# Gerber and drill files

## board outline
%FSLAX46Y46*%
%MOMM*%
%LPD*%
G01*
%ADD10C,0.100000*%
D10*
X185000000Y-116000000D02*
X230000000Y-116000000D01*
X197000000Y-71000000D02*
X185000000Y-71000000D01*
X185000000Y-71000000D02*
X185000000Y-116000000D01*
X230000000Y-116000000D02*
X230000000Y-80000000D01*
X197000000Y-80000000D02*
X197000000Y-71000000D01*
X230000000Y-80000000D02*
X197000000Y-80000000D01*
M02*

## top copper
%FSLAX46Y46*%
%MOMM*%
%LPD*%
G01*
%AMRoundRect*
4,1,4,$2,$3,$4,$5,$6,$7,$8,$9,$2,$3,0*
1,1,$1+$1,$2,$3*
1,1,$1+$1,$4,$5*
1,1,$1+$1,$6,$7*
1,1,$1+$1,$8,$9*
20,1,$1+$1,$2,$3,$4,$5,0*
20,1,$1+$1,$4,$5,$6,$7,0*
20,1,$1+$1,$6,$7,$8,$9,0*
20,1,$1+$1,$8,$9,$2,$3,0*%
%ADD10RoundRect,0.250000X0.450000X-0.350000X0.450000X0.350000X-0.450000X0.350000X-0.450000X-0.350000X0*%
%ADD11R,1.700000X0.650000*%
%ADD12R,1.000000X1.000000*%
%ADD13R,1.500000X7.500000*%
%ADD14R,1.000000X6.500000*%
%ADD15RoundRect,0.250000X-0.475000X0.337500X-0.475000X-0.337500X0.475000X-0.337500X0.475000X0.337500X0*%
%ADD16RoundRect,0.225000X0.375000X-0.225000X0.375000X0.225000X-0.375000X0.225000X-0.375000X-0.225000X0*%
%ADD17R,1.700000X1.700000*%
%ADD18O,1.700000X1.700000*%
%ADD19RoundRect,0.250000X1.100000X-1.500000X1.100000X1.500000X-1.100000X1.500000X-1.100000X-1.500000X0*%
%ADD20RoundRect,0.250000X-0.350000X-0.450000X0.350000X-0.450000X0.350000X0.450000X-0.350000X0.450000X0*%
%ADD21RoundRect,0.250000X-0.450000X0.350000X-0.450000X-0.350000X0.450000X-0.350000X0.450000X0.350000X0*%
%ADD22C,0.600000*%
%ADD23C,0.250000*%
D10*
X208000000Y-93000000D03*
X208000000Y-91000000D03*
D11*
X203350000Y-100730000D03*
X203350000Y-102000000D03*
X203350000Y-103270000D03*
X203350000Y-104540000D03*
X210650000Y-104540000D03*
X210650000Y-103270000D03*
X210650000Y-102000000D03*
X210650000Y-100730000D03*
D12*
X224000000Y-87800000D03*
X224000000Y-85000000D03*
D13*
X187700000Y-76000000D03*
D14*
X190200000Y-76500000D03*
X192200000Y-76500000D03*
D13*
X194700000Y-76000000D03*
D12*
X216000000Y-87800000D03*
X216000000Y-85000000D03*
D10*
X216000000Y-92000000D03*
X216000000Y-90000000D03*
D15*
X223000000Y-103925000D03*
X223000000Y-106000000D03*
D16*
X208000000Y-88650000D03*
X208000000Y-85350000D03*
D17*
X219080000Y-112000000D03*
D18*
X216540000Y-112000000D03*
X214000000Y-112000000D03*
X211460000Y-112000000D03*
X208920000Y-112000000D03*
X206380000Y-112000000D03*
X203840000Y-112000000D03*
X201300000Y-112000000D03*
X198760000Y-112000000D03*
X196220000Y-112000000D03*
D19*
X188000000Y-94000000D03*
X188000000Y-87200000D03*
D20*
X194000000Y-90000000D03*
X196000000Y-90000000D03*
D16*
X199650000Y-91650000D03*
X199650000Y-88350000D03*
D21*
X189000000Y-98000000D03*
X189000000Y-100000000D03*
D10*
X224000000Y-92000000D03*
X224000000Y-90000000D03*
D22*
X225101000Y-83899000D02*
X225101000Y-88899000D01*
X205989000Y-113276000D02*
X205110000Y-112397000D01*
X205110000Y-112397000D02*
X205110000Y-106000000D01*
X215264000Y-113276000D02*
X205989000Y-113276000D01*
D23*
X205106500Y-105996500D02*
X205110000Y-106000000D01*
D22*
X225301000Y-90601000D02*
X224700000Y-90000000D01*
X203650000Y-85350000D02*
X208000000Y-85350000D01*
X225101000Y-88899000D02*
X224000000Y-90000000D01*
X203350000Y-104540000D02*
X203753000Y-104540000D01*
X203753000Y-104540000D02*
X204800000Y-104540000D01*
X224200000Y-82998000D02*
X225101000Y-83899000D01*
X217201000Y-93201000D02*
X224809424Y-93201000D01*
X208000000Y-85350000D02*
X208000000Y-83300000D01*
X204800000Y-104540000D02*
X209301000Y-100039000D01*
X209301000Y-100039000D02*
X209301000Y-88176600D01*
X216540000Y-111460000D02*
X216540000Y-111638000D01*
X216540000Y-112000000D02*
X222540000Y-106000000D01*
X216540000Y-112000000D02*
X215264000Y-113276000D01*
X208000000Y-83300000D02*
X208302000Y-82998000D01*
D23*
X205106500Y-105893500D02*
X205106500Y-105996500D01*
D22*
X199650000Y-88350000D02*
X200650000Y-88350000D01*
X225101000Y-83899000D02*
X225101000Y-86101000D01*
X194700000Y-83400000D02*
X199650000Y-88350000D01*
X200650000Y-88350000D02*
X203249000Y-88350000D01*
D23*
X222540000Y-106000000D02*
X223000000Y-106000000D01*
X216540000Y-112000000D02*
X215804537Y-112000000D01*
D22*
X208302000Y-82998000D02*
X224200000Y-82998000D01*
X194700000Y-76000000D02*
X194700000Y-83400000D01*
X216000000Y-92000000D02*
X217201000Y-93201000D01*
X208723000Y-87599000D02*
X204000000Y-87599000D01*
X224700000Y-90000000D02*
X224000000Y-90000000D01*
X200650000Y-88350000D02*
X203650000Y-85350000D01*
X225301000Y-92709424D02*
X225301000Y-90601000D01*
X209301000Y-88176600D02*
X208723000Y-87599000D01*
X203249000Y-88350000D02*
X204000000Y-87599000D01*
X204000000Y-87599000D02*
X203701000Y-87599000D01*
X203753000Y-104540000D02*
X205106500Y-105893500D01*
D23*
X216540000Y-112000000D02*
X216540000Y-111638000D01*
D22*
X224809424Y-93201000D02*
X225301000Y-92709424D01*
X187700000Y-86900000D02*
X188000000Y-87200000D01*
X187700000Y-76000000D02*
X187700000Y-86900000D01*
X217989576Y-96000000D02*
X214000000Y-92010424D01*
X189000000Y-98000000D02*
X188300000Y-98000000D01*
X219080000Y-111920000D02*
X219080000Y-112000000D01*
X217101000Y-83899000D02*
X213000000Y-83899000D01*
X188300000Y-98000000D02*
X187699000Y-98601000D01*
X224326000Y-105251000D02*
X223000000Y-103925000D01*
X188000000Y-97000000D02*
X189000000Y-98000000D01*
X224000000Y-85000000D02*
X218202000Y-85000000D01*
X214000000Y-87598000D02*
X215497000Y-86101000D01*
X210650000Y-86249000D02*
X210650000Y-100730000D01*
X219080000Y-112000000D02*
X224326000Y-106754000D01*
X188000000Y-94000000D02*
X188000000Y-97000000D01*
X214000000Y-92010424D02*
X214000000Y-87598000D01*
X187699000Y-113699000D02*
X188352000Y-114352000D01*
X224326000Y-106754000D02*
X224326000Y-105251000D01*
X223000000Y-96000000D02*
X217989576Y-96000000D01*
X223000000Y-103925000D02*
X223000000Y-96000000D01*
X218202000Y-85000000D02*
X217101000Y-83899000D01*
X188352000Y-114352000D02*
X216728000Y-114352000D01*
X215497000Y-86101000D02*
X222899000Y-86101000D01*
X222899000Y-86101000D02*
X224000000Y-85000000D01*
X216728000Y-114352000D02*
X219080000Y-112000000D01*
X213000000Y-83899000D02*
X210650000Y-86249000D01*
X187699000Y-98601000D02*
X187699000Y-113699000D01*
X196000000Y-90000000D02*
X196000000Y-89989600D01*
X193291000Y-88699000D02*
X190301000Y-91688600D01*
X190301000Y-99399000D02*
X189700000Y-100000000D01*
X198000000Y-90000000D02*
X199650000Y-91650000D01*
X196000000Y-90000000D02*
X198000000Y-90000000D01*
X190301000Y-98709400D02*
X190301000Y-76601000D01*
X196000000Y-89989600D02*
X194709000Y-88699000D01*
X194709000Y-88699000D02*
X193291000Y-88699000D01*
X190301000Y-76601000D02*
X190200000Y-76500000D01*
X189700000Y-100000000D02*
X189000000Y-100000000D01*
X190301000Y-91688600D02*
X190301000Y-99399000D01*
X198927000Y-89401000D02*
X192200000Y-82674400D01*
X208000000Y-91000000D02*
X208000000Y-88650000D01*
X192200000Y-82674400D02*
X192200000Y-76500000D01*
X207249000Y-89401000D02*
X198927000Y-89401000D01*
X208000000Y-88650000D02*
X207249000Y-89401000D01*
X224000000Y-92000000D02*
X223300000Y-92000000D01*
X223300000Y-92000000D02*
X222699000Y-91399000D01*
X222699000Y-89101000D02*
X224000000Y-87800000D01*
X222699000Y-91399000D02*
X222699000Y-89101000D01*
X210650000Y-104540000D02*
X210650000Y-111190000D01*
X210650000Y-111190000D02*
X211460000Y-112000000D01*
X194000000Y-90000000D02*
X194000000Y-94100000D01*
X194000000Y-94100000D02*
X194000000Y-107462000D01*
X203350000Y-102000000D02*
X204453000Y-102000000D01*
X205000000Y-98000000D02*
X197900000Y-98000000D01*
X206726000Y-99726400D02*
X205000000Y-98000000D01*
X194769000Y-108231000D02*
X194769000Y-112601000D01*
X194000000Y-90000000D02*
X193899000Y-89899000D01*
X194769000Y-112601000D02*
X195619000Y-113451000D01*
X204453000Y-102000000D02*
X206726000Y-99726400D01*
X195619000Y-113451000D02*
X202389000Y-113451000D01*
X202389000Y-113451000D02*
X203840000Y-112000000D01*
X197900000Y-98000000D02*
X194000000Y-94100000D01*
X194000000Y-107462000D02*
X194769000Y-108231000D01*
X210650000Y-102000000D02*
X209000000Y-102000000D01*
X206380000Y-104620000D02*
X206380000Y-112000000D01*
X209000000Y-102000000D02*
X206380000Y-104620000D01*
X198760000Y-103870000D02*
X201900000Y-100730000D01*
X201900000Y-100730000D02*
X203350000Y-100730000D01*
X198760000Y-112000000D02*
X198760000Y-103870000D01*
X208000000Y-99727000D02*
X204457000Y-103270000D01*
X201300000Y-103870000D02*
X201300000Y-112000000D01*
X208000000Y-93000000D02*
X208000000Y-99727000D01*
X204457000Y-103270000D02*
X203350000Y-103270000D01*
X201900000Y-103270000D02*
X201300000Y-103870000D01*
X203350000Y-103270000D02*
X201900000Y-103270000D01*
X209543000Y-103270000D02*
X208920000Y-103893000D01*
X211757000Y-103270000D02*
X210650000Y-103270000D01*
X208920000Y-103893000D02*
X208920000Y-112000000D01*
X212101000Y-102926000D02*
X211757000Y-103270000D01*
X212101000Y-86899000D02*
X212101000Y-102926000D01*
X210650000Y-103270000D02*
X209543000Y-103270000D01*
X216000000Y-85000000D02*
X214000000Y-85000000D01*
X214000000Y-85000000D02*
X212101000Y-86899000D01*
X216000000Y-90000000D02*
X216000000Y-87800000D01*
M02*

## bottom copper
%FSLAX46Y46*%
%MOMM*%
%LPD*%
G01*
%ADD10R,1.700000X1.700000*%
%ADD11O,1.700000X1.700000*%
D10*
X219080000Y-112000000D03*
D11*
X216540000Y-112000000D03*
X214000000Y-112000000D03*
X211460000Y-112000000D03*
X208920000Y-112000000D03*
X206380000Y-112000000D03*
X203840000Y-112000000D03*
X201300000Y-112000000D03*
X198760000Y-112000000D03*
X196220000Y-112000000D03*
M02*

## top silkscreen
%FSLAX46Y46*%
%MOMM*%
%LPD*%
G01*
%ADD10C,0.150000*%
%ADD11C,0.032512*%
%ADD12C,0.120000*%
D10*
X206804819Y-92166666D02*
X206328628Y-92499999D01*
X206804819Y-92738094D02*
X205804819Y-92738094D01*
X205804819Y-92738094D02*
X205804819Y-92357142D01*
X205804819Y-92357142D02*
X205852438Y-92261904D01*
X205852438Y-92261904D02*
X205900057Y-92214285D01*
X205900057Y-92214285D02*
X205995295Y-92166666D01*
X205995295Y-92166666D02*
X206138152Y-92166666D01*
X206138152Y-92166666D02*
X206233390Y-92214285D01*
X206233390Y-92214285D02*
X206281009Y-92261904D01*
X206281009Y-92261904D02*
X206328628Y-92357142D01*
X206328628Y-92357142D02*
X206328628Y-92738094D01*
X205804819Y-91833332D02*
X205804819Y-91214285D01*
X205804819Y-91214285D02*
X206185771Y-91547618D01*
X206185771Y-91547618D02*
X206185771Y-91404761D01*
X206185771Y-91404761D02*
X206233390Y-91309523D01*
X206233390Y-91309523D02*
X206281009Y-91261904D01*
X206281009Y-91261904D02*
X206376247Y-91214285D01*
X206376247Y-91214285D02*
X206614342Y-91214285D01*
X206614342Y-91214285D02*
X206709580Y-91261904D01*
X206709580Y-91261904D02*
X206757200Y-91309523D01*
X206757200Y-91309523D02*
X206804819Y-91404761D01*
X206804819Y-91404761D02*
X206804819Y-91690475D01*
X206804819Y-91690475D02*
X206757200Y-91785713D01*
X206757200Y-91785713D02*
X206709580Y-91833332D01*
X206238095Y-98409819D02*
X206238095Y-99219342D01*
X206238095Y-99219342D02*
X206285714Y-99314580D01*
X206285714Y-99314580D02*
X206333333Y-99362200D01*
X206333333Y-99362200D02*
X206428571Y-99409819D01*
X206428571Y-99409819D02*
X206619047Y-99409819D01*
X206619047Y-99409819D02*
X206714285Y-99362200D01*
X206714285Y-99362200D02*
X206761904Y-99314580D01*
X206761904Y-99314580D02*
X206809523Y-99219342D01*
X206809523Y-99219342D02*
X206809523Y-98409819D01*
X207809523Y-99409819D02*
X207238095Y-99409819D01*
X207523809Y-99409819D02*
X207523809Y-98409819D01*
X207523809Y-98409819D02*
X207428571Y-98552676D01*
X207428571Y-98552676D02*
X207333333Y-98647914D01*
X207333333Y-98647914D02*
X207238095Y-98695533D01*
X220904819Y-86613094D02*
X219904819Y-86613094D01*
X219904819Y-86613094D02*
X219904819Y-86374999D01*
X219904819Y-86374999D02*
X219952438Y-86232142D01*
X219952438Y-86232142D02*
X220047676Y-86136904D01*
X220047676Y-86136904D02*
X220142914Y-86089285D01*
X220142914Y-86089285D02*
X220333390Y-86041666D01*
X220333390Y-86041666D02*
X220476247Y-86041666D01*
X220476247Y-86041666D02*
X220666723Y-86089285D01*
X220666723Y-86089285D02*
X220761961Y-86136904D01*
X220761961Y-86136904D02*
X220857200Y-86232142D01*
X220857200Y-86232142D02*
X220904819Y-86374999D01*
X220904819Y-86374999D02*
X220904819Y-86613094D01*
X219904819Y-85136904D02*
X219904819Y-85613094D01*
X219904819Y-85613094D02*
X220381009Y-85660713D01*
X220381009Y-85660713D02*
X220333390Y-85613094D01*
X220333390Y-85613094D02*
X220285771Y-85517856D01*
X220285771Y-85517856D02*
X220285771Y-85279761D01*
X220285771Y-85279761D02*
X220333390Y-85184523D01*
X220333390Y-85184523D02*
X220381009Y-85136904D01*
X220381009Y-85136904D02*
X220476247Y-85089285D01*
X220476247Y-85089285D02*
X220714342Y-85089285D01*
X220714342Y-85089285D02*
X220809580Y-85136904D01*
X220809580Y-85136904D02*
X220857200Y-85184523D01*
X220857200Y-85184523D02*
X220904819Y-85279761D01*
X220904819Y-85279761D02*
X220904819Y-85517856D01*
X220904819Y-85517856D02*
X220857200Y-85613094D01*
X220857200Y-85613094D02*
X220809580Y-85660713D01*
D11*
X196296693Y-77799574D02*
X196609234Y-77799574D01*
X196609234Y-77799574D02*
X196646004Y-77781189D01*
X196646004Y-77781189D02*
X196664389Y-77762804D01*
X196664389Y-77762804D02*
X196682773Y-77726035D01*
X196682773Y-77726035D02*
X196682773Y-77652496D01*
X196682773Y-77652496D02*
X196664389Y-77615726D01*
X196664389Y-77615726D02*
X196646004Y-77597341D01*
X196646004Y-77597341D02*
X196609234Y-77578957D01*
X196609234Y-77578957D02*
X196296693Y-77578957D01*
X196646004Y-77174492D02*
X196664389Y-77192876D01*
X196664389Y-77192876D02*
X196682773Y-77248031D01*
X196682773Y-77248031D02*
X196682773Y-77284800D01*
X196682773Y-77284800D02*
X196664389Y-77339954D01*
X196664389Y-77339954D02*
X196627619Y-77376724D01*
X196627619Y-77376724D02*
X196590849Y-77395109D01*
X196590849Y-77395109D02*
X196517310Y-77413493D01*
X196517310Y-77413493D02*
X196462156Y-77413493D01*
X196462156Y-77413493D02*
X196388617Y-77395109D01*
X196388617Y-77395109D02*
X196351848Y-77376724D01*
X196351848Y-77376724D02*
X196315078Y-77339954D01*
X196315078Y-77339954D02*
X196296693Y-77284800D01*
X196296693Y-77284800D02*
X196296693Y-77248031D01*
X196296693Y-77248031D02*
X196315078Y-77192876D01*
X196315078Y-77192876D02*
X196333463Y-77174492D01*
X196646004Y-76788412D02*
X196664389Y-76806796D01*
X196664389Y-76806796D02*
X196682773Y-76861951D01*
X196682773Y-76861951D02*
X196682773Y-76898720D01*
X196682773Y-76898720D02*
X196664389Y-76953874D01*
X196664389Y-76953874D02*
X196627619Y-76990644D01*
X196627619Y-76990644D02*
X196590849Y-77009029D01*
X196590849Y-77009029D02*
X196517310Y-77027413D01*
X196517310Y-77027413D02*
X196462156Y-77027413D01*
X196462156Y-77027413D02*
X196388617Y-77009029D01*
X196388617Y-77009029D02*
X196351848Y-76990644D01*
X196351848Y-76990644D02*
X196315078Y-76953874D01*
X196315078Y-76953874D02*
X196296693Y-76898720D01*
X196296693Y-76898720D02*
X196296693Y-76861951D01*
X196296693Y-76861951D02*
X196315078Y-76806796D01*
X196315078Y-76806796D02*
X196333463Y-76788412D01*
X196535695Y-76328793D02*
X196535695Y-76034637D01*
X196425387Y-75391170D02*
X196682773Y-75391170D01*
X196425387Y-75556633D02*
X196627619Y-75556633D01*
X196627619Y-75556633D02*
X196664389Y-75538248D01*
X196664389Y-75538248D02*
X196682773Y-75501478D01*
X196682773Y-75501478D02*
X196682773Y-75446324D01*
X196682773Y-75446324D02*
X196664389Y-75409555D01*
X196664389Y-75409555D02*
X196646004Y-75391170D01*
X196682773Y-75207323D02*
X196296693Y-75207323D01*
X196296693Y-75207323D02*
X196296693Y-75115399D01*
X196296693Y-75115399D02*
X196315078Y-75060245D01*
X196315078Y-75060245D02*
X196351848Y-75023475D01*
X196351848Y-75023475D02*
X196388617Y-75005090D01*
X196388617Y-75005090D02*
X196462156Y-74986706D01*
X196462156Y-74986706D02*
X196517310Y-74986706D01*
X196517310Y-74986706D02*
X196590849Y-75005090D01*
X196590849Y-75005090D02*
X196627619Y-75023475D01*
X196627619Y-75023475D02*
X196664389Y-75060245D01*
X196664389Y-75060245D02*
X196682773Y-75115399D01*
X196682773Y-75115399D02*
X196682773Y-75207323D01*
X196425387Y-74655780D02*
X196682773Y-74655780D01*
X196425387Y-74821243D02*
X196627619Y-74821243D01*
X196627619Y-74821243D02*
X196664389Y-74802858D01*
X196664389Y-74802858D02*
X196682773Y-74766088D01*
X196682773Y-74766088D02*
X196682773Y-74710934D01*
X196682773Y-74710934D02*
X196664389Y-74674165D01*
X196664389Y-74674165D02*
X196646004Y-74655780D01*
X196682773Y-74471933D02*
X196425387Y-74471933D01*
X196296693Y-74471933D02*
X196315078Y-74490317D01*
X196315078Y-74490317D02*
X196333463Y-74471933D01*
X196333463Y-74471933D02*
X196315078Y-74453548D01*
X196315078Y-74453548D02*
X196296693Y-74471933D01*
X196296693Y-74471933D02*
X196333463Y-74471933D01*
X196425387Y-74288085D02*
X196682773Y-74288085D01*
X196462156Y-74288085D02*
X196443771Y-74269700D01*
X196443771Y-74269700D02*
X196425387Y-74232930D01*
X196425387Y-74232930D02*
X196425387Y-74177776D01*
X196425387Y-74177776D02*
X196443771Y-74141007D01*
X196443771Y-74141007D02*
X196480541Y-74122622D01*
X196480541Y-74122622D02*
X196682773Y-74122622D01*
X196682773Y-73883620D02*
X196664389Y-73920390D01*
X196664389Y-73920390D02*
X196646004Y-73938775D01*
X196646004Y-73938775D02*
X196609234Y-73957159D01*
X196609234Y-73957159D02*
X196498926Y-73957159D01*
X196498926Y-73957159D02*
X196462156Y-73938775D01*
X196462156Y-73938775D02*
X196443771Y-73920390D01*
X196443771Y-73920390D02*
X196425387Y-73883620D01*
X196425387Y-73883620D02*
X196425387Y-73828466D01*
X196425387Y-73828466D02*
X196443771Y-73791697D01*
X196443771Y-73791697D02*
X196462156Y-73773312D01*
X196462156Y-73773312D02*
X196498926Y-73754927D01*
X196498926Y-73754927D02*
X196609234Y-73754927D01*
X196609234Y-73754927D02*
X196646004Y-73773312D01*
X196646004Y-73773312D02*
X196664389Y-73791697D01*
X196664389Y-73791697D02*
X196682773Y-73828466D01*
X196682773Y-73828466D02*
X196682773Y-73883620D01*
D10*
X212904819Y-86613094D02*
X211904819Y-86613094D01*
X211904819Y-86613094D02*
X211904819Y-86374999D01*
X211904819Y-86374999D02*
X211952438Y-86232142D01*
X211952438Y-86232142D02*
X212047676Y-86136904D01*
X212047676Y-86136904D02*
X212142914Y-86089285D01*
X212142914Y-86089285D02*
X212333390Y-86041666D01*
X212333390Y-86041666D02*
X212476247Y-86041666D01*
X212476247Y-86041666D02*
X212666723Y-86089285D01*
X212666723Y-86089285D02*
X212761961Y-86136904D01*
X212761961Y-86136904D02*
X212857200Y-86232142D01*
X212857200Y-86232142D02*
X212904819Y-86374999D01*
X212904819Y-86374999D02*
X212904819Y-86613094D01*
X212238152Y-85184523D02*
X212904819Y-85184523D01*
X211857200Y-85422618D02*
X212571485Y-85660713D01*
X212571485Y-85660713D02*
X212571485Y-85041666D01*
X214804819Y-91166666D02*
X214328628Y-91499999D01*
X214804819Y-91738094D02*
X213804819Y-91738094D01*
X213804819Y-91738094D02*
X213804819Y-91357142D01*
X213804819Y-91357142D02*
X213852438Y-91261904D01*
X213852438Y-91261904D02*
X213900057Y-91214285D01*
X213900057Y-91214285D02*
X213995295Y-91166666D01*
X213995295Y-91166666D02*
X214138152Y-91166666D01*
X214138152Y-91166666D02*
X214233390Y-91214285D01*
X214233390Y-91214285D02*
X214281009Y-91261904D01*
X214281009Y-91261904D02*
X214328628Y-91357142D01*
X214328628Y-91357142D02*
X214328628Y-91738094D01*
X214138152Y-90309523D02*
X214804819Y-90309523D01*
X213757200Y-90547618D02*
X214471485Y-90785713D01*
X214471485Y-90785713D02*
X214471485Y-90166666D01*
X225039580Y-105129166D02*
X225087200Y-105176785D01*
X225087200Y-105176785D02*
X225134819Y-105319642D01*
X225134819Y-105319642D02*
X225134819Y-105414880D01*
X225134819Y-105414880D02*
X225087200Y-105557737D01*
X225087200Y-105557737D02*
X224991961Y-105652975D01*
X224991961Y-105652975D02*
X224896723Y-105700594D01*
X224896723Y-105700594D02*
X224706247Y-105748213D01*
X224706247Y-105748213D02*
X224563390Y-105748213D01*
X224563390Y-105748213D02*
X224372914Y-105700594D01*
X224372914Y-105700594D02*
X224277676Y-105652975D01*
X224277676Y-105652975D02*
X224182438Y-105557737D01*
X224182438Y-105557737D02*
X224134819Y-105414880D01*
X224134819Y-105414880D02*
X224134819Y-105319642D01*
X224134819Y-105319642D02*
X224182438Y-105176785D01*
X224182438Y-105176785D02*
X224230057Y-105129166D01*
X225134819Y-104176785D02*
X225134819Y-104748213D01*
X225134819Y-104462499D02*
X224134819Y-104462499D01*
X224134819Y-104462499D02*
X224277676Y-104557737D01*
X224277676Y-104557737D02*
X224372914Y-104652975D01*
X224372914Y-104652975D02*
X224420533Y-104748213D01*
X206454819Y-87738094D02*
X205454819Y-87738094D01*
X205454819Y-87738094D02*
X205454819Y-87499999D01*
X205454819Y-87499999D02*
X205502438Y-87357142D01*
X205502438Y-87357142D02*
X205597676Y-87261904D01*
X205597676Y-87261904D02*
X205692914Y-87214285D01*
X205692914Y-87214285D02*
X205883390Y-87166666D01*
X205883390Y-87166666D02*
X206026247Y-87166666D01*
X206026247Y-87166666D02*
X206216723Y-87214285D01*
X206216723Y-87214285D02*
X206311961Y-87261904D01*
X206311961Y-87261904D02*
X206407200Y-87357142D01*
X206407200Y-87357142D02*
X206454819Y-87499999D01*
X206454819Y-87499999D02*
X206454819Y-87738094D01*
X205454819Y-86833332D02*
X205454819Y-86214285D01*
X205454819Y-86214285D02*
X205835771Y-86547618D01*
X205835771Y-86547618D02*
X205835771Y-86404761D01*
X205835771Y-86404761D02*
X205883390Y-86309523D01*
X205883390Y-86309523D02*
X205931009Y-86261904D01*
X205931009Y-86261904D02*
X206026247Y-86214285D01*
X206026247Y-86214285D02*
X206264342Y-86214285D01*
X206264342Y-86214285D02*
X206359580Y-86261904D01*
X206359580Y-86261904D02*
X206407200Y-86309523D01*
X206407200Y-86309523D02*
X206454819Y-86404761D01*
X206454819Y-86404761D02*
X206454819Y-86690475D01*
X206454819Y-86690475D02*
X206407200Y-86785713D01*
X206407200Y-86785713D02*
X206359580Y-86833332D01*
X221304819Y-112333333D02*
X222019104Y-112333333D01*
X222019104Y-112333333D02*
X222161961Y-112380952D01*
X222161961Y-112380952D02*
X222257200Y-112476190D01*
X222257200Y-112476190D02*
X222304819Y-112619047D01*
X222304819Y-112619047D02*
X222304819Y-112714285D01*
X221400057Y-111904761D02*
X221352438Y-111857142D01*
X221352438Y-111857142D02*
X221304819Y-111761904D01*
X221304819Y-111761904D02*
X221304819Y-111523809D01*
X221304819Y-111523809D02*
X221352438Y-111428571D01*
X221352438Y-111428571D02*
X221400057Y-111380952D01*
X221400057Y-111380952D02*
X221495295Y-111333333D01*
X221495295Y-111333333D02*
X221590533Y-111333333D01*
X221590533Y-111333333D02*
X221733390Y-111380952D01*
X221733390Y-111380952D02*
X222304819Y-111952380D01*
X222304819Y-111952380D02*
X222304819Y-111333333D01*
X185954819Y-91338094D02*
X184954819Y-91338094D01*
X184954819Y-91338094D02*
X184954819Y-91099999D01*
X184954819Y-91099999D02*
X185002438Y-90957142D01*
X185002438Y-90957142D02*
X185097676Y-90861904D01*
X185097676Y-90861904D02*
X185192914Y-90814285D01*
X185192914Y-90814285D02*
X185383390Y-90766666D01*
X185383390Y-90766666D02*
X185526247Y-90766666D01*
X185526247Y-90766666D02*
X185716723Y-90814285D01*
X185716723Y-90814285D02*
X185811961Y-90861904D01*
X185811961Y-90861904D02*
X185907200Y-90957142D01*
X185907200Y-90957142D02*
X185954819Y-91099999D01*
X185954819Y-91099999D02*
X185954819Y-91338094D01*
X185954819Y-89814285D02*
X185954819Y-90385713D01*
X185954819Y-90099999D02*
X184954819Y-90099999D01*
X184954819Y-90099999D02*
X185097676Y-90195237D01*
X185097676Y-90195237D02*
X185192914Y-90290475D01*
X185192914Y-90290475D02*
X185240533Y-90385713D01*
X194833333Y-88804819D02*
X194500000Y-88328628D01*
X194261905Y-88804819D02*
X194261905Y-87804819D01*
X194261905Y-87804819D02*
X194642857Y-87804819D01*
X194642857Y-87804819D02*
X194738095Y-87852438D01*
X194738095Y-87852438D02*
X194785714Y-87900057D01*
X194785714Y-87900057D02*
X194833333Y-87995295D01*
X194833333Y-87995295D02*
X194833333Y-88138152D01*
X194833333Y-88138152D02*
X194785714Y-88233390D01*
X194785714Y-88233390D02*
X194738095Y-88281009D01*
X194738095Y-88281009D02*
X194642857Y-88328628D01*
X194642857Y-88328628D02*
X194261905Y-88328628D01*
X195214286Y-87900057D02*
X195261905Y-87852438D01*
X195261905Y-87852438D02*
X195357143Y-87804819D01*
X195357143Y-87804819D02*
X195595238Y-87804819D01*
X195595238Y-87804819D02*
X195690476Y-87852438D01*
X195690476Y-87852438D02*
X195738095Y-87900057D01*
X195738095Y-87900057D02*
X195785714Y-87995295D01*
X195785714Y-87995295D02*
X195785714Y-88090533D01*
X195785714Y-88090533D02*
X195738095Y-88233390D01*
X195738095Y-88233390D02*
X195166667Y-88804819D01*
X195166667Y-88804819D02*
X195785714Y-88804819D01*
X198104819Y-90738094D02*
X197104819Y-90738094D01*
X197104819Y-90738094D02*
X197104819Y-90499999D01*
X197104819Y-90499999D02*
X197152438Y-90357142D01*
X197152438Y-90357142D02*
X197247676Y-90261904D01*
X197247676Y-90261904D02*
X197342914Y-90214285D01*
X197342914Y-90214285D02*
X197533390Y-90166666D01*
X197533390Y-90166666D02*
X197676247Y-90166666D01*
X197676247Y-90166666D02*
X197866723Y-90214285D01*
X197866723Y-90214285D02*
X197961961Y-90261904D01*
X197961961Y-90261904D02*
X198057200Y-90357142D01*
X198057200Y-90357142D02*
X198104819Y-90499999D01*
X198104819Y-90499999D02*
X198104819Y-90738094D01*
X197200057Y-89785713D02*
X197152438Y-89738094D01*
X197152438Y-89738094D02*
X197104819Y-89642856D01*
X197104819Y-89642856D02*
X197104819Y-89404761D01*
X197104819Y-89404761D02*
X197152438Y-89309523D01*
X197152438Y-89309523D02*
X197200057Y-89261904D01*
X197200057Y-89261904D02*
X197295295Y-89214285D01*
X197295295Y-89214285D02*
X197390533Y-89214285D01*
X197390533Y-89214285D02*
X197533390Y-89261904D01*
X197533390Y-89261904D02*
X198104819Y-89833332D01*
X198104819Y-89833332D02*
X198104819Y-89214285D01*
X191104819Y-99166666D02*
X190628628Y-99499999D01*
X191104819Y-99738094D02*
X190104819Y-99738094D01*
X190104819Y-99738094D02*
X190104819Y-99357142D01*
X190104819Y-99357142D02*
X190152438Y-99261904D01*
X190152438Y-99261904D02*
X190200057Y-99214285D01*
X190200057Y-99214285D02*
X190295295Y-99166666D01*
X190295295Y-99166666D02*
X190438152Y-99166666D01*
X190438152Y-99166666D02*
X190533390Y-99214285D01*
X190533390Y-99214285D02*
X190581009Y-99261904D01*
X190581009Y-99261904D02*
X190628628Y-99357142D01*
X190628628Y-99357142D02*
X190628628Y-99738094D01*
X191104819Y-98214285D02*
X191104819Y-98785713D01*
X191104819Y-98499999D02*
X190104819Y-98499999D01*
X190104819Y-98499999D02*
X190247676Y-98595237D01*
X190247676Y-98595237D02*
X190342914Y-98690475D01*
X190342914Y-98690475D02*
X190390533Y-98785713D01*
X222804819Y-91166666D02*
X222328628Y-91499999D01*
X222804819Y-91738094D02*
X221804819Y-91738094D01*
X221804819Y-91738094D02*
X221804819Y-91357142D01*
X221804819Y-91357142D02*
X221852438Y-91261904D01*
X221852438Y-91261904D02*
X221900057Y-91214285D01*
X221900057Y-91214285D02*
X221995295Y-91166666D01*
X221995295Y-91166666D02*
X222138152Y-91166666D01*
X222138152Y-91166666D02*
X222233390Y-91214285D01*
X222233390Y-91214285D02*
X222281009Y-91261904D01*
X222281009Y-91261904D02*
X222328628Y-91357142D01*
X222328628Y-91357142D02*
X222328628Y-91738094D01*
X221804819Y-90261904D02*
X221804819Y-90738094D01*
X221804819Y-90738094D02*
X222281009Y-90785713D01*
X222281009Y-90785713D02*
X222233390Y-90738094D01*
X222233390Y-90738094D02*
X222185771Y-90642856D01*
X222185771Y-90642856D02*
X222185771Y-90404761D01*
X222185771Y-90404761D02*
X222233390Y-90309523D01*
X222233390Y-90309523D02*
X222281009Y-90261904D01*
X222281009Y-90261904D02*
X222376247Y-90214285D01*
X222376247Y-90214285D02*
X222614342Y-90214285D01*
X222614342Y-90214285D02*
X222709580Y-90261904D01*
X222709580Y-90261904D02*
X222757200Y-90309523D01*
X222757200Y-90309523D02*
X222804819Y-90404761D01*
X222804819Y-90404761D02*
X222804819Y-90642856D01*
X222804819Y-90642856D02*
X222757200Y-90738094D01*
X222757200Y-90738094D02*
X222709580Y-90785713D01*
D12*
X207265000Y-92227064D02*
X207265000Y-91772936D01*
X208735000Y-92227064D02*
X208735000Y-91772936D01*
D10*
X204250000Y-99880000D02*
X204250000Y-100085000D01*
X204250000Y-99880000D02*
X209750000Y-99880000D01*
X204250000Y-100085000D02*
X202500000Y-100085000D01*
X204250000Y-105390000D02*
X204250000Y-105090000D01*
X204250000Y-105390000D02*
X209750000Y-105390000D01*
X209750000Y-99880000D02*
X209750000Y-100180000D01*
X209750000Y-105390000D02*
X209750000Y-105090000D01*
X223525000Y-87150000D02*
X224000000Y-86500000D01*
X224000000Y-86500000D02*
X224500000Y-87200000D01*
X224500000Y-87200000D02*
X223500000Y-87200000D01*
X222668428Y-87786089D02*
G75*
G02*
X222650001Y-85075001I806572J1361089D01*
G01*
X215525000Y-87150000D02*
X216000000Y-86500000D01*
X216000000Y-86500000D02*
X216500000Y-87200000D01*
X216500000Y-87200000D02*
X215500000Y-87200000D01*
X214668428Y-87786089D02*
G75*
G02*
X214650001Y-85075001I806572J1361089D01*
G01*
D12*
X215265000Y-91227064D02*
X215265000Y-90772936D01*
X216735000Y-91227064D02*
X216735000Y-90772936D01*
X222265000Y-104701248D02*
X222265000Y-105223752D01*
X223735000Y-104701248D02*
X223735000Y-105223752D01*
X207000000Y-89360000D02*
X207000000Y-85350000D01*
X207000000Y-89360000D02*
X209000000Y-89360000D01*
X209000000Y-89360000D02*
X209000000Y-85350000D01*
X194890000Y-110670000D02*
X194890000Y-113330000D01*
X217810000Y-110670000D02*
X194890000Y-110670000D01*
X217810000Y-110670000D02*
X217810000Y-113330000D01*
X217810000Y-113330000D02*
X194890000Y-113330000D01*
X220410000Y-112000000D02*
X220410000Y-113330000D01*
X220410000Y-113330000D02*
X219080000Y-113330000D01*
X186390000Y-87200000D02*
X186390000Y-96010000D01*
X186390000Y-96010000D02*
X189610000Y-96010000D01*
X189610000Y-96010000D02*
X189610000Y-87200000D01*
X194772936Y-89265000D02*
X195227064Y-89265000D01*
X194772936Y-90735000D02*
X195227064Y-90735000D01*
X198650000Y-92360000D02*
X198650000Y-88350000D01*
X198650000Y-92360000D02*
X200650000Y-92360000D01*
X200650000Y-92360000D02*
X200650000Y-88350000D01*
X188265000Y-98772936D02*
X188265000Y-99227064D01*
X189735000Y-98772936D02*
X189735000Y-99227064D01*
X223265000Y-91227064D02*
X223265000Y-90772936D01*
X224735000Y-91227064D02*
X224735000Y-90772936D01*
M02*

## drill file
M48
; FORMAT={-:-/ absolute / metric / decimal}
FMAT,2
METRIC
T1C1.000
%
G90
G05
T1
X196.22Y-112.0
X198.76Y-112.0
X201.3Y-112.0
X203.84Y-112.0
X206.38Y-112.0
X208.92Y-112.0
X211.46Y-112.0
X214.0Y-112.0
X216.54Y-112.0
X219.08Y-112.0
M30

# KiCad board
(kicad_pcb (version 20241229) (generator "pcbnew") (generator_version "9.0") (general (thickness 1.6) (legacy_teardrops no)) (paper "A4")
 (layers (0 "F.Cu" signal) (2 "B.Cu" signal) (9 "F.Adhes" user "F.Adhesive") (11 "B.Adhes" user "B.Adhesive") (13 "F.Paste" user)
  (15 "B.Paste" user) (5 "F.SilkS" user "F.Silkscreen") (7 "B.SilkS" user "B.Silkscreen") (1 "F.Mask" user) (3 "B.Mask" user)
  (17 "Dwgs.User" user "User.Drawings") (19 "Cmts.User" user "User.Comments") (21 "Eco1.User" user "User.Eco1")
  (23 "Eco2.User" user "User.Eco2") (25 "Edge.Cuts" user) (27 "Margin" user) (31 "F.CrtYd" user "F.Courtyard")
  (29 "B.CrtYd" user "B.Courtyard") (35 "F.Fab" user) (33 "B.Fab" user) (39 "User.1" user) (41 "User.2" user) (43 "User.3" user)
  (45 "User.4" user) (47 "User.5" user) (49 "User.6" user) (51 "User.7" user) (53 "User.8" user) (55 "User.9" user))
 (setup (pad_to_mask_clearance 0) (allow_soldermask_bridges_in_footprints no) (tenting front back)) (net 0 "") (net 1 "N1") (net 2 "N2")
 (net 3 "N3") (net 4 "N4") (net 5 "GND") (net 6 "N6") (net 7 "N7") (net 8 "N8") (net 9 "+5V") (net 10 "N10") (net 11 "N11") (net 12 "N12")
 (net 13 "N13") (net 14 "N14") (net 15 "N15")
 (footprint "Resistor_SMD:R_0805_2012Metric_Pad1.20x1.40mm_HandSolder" (layer "F.Cu") (at 208 92 90)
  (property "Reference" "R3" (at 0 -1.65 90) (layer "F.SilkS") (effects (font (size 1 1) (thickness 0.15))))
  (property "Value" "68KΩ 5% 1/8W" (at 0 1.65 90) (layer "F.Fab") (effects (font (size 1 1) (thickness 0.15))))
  (fp_line (start -0.227064 -0.735) (end 0.227064 -0.735) (stroke (width 0.12) (type solid)) (layer "F.SilkS"))
  (fp_line (start -0.227064 0.735) (end 0.227064 0.735) (stroke (width 0.12) (type solid)) (layer "F.SilkS"))
  (pad "1" smd roundrect (at -1 0 90) (size 1.2 1.4) (layers "F.Cu" "F.Mask" "F.Paste") (roundrect_rratio 0.208333) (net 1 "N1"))
  (pad "2" smd roundrect (at 1 0 90) (size 1.2 1.4) (layers "F.Cu" "F.Mask" "F.Paste") (roundrect_rratio 0.208333) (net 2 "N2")))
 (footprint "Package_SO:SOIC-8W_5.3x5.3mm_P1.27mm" (layer "F.Cu") (at 207 102.635)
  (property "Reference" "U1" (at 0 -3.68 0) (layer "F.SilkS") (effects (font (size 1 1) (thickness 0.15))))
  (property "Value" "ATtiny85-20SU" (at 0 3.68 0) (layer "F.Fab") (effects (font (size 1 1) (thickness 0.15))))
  (fp_line (start -2.75 -2.755) (end -2.75 -2.55) (stroke (width 0.15) (type solid)) (layer "F.SilkS"))
  (fp_line (start -2.75 -2.755) (end 2.75 -2.755) (stroke (width 0.15) (type solid)) (layer "F.SilkS"))
  (fp_line (start -2.75 -2.55) (end -4.5 -2.55) (stroke (width 0.15) (type solid)) (layer "F.SilkS"))
  (fp_line (start -2.75 2.755) (end -2.75 2.455) (stroke (width 0.15) (type solid)) (layer "F.SilkS"))
  (fp_line (start -2.75 2.755) (end 2.75 2.755) (stroke (width 0.15) (type solid)) (layer "F.SilkS"))
  (fp_line (start 2.75 -2.755) (end 2.75 -2.455) (stroke (width 0.15) (type solid)) (layer "F.SilkS"))
  (fp_line (start 2.75 2.755) (end 2.75 2.455) (stroke (width 0.15) (type solid)) (layer "F.SilkS"))
  (pad "1" smd rect (at -3.65 -1.905) (size 1.7 0.65) (layers "F.Cu" "F.Mask" "F.Paste") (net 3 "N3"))
  (pad "2" smd rect (at -3.65 -0.635) (size 1.7 0.65) (layers "F.Cu" "F.Mask" "F.Paste") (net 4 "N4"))
  (pad "3" smd rect (at -3.65 0.635) (size 1.7 0.65) (layers "F.Cu" "F.Mask" "F.Paste") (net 1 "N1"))
  (pad "4" smd rect (at -3.65 1.905) (size 1.7 0.65) (layers "F.Cu" "F.Mask" "F.Paste") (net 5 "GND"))
  (pad "5" smd rect (at 3.65 1.905) (size 1.7 0.65) (layers "F.Cu" "F.Mask" "F.Paste") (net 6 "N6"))
  (pad "6" smd rect (at 3.65 0.635) (size 1.7 0.65) (layers "F.Cu" "F.Mask" "F.Paste") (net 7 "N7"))
  (pad "7" smd rect (at 3.65 -0.635) (size 1.7 0.65) (layers "F.Cu" "F.Mask" "F.Paste") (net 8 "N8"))
  (pad "8" smd rect (at 3.65 -1.905) (size 1.7 0.65) (layers "F.Cu" "F.Mask" "F.Paste") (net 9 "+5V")))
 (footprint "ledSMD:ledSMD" (layer "F.Cu") (at 224 86 90)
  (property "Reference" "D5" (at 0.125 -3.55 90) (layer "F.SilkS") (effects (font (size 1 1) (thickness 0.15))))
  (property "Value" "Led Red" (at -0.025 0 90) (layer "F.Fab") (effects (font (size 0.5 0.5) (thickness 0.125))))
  (fp_line (start -1.15 -0.475) (end -0.5 0) (stroke (width 0.15) (type solid)) (layer "F.SilkS"))
  (fp_line (start -0.5 0) (end -1.2 0.5) (stroke (width 0.15) (type solid)) (layer "F.SilkS"))
  (fp_line (start -1.2 0.5) (end -1.2 -0.5) (stroke (width 0.15) (type solid)) (layer "F.SilkS"))
  (fp_arc (start -1.786089 -1.331572) (mid -0.435753 -2.107089) (end 0.924999 -1.349999) (stroke (width 0.15) (type solid))
   (layer "F.SilkS"))
  (pad "1" smd rect (at -1.8 0 90) (size 1 1) (layers "F.Cu" "F.Mask" "F.Paste") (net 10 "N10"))
  (pad "2" smd rect (at 1 0 90) (size 1 1) (layers "F.Cu" "F.Mask" "F.Paste") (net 9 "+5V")))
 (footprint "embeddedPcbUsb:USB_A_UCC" (layer "F.Cu") (at 191.2 76.2 -90)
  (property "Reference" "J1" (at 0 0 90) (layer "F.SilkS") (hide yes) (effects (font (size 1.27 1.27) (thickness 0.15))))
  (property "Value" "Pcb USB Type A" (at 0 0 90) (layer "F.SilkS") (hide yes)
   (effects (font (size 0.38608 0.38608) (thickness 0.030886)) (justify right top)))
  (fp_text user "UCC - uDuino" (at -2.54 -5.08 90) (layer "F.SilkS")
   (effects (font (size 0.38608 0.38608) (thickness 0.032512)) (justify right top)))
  (pad "1" smd rect (at -0.2 3.5 270) (size 7.5 1.5) (layers "F.Cu" "F.Mask" "F.Paste") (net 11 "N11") (solder_mask_margin 0.1016))
  (pad "2" smd rect (at 0.3 1 270) (size 6.5 1) (layers "F.Cu" "F.Mask" "F.Paste") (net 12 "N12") (solder_mask_margin 0.1016))
  (pad "3" smd rect (at 0.3 -1 270) (size 6.5 1) (layers "F.Cu" "F.Mask" "F.Paste") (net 2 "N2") (solder_mask_margin 0.1016))
  (pad "4" smd rect (at -0.2 -3.5 270) (size 7.5 1.5) (layers "F.Cu" "F.Mask" "F.Paste") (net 5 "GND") (solder_mask_margin 0.1016)))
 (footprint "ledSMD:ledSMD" (layer "F.Cu") (at 216 86 90)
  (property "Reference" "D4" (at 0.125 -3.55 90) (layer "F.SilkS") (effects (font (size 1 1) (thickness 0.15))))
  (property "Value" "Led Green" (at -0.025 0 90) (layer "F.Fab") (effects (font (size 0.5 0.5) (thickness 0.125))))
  (fp_line (start -1.15 -0.475) (end -0.5 0) (stroke (width 0.15) (type solid)) (layer "F.SilkS"))
  (fp_line (start -0.5 0) (end -1.2 0.5) (stroke (width 0.15) (type solid)) (layer "F.SilkS"))
  (fp_line (start -1.2 0.5) (end -1.2 -0.5) (stroke (width 0.15) (type solid)) (layer "F.SilkS"))
  (fp_arc (start -1.786089 -1.331572) (mid -0.435753 -2.107089) (end 0.924999 -1.349999) (stroke (width 0.15) (type solid))
   (layer "F.SilkS"))
  (pad "1" smd rect (at -1.8 0 90) (size 1 1) (layers "F.Cu" "F.Mask" "F.Paste") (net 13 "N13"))
  (pad "2" smd rect (at 1 0 90) (size 1 1) (layers "F.Cu" "F.Mask" "F.Paste") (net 7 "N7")))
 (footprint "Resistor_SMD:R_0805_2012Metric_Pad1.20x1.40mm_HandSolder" (layer "F.Cu") (at 216 91 90)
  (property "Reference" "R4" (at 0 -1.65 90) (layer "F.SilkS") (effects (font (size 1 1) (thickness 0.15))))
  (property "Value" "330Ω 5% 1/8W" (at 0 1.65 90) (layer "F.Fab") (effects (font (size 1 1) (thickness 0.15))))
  (fp_line (start -0.227064 -0.735) (end 0.227064 -0.735) (stroke (width 0.12) (type solid)) (layer "F.SilkS"))
  (fp_line (start -0.227064 0.735) (end 0.227064 0.735) (stroke (width 0.12) (type solid)) (layer "F.SilkS"))
  (pad "1" smd roundrect (at -1 0 90) (size 1.2 1.4) (layers "F.Cu" "F.Mask" "F.Paste") (roundrect_rratio 0.208333) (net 5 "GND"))
  (pad "2" smd roundrect (at 1 0 90) (size 1.2 1.4) (layers "F.Cu" "F.Mask" "F.Paste") (roundrect_rratio 0.208333) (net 13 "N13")))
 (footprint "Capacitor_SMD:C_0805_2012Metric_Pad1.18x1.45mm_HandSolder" (layer "F.Cu") (at 223 104.9625 -90)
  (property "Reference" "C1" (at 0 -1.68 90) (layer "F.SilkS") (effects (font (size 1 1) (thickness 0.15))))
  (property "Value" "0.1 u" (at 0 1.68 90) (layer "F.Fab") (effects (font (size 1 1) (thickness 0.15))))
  (fp_line (start -0.261252 0.735) (end 0.261252 0.735) (stroke (width 0.12) (type solid)) (layer "F.SilkS"))
  (fp_line (start -0.261252 -0.735) (end 0.261252 -0.735) (stroke (width 0.12) (type solid)) (layer "F.SilkS"))
  (pad "1" smd roundrect (at -1.0375 0 270) (size 1.175 1.45) (layers "F.Cu" "F.Mask" "F.Paste") (roundrect_rratio 0.212766) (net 9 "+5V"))
  (pad "2" smd roundrect (at 1.0375 0 270) (size 1.175 1.45) (layers "F.Cu" "F.Mask" "F.Paste") (roundrect_rratio 0.212766) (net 5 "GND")))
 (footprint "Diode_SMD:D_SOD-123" (layer "F.Cu") (at 208 87 90)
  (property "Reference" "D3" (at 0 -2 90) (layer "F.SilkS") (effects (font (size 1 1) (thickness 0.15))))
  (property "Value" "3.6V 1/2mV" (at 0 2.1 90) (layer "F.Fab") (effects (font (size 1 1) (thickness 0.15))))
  (fp_line (start -2.36 -1) (end 1.65 -1) (stroke (width 0.12) (type solid)) (layer "F.SilkS"))
  (fp_line (start -2.36 -1) (end -2.36 1) (stroke (width 0.12) (type solid)) (layer "F.SilkS"))
  (fp_line (start -2.36 1) (end 1.65 1) (stroke (width 0.12) (type solid)) (layer "F.SilkS"))
  (pad "1" smd roundrect (at -1.65 0 90) (size 0.9 1.2) (layers "F.Cu" "F.Mask" "F.Paste") (roundrect_rratio 0.25) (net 2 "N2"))
  (pad "2" smd roundrect (at 1.65 0 90) (size 0.9 1.2) (layers "F.Cu" "F.Mask" "F.Paste") (roundrect_rratio 0.25) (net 5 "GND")))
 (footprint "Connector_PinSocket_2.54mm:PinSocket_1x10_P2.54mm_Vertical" (layer "F.Cu") (at 219.08 112 -90)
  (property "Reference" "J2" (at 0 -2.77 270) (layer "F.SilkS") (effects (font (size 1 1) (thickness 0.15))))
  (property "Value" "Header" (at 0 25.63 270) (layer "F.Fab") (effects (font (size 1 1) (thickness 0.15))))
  (fp_line (start -1.33 24.19) (end 1.33 24.19) (stroke (width 0.12) (type solid)) (layer "F.SilkS"))
  (fp_line (start -1.33 1.27) (end -1.33 24.19) (stroke (width 0.12) (type solid)) (layer "F.SilkS"))
  (fp_line (start -1.33 1.27) (end 1.33 1.27) (stroke (width 0.12) (type solid)) (layer "F.SilkS"))
  (fp_line (start 1.33 1.27) (end 1.33 24.19) (stroke (width 0.12) (type solid)) (layer "F.SilkS"))
  (fp_line (start 0 -1.33) (end 1.33 -1.33) (stroke (width 0.12) (type solid)) (layer "F.SilkS"))
  (fp_line (start 1.33 -1.33) (end 1.33 0) (stroke (width 0.12) (type solid)) (layer "F.SilkS"))
  (pad "1" thru_hole rect (at 0 0 270) (size 1.7 1.7) (drill 1) (layers "*.Cu" "*.Mask") (remove_unused_layers no) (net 9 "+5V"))
  (pad "2" thru_hole oval (at 0 2.54 270) (size 1.7 1.7) (drill 1) (layers "*.Cu" "*.Mask") (remove_unused_layers no) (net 5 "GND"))
  (pad "3" thru_hole oval (at 0 5.08 270) (size 1.7 1.7) (drill 1) (layers "*.Cu" "*.Mask") (remove_unused_layers no) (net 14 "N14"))
  (pad "4" thru_hole oval (at 0 7.62 270) (size 1.7 1.7) (drill 1) (layers "*.Cu" "*.Mask") (remove_unused_layers no) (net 6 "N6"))
  (pad "5" thru_hole oval (at 0 10.16 270) (size 1.7 1.7) (drill 1) (layers "*.Cu" "*.Mask") (remove_unused_layers no) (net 7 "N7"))
  (pad "6" thru_hole oval (at 0 12.7 270) (size 1.7 1.7) (drill 1) (layers "*.Cu" "*.Mask") (remove_unused_layers no) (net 8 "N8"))
  (pad "7" thru_hole oval (at 0 15.24 270) (size 1.7 1.7) (drill 1) (layers "*.Cu" "*.Mask") (remove_unused_layers no) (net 4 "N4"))
  (pad "8" thru_hole oval (at 0 17.78 270) (size 1.7 1.7) (drill 1) (layers "*.Cu" "*.Mask") (remove_unused_layers no) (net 1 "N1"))
  (pad "9" thru_hole oval (at 0 20.32 270) (size 1.7 1.7) (drill 1) (layers "*.Cu" "*.Mask") (remove_unused_layers no) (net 3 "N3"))
  (pad "10" thru_hole oval (at 0 22.86 270) (size 1.7 1.7) (drill 1) (layers "*.Cu" "*.Mask") (remove_unused_layers no) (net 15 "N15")))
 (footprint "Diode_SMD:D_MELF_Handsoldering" (layer "F.Cu") (at 188 90.6 90)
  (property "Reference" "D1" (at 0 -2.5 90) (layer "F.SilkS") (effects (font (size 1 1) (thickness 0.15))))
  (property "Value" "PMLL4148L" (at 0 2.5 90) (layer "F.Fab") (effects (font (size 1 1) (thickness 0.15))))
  (fp_line (start 3.4 -1.61) (end -5.41 -1.61) (stroke (width 0.12) (type solid)) (layer "F.SilkS"))
  (fp_line (start -5.41 -1.61) (end -5.41 1.61) (stroke (width 0.12) (type solid)) (layer "F.SilkS"))
  (fp_line (start -5.41 1.61) (end 3.4 1.61) (stroke (width 0.12) (type solid)) (layer "F.SilkS"))
  (pad "1" smd roundrect (at -3.4 0 90) (size 3.5 2.7) (layers "F.Cu" "F.Mask" "F.Paste") (roundrect_rratio 0.0925925926) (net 9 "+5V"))
  (pad "2" smd roundrect (at 3.4 0 90) (size 3.5 2.7) (layers "F.Cu" "F.Mask" "F.Paste") (roundrect_rratio 0.0925925926) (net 11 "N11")))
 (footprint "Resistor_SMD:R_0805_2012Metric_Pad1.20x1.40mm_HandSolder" (layer "F.Cu") (at 195 90)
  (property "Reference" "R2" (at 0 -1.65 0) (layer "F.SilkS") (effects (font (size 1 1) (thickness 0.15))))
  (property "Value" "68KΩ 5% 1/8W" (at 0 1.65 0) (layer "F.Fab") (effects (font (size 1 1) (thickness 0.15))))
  (fp_line (start -0.227064 -0.735) (end 0.227064 -0.735) (stroke (width 0.12) (type solid)) (layer "F.SilkS"))
  (fp_line (start -0.227064 0.735) (end 0.227064 0.735) (stroke (width 0.12) (type solid)) (layer "F.SilkS"))
  (pad "1" smd roundrect (at -1 0) (size 1.2 1.4) (layers "F.Cu" "F.Mask" "F.Paste") (roundrect_rratio 0.208333) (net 4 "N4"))
  (pad "2" smd roundrect (at 1 0) (size 1.2 1.4) (layers "F.Cu" "F.Mask" "F.Paste") (roundrect_rratio 0.208333) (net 12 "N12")))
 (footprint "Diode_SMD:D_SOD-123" (layer "F.Cu") (at 199.65 90 90)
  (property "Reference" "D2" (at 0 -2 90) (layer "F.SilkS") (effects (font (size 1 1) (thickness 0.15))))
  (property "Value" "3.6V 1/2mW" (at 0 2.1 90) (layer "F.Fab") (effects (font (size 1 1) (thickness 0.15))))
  (fp_line (start -2.36 -1) (end 1.65 -1) (stroke (width 0.12) (type solid)) (layer "F.SilkS"))
  (fp_line (start -2.36 -1) (end -2.36 1) (stroke (width 0.12) (type solid)) (layer "F.SilkS"))
  (fp_line (start -2.36 1) (end 1.65 1) (stroke (width 0.12) (type solid)) (layer "F.SilkS"))
  (pad "1" smd roundrect (at -1.65 0 90) (size 0.9 1.2) (layers "F.Cu" "F.Mask" "F.Paste") (roundrect_rratio 0.25) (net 12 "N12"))
  (pad "2" smd roundrect (at 1.65 0 90) (size 0.9 1.2) (layers "F.Cu" "F.Mask" "F.Paste") (roundrect_rratio 0.25) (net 5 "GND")))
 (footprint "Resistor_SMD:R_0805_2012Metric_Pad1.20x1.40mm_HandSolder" (layer "F.Cu") (at 189 99 -90)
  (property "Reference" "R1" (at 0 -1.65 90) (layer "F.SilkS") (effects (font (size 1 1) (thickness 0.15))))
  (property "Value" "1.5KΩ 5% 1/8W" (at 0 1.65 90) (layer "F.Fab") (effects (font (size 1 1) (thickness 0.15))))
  (fp_line (start -0.227064 0.735) (end 0.227064 0.735) (stroke (width 0.12) (type solid)) (layer "F.SilkS"))
  (fp_line (start -0.227064 -0.735) (end 0.227064 -0.735) (stroke (width 0.12) (type solid)) (layer "F.SilkS"))
  (pad "1" smd roundrect (at -1 0 270) (size 1.2 1.4) (layers "F.Cu" "F.Mask" "F.Paste") (roundrect_rratio 0.208333) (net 9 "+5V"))
  (pad "2" smd roundrect (at 1 0 270) (size 1.2 1.4) (layers "F.Cu" "F.Mask" "F.Paste") (roundrect_rratio 0.208333) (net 12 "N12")))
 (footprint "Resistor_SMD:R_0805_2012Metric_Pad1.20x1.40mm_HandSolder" (layer "F.Cu") (at 224 91 90)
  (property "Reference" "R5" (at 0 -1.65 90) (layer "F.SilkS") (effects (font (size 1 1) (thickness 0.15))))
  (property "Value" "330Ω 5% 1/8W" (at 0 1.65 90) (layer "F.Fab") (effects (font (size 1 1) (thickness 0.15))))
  (fp_line (start -0.227064 -0.735) (end 0.227064 -0.735) (stroke (width 0.12) (type solid)) (layer "F.SilkS"))
  (fp_line (start -0.227064 0.735) (end 0.227064 0.735) (stroke (width 0.12) (type solid)) (layer "F.SilkS"))
  (pad "1" smd roundrect (at -1 0 90) (size 1.2 1.4) (layers "F.Cu" "F.Mask" "F.Paste") (roundrect_rratio 0.208333) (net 10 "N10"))
  (pad "2" smd roundrect (at 1 0 90) (size 1.2 1.4) (layers "F.Cu" "F.Mask" "F.Paste") (roundrect_rratio 0.208333) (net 5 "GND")))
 (gr_line (start 185 116) (end 230 116) (stroke (width 0.1) (type default)) (layer "Edge.Cuts"))
 (gr_line (start 197 71) (end 185 71) (stroke (width 0.1) (type default)) (layer "Edge.Cuts"))
 (gr_line (start 185 71) (end 185 116) (stroke (width 0.1) (type default)) (layer "Edge.Cuts"))
 (gr_line (start 230 116) (end 230 80) (stroke (width 0.1) (type default)) (layer "Edge.Cuts"))
 (gr_line (start 197 80) (end 197 71) (stroke (width 0.1) (type default)) (layer "Edge.Cuts"))
 (gr_line (start 230 80) (end 197 80) (stroke (width 0.1) (type default)) (layer "Edge.Cuts"))
 (segment (start 225.101 83.899) (end 225.101 88.899) (width 0.6) (layer "F.Cu") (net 5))
 (segment (start 205.989 113.276) (end 205.11 112.397) (width 0.6) (layer "F.Cu") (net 5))
 (segment (start 205.11 112.397) (end 205.11 106) (width 0.6) (layer "F.Cu") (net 5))
 (segment (start 215.264 113.276) (end 205.989 113.276) (width 0.6) (layer "F.Cu") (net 5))
 (segment (start 205.1065 105.9965) (end 205.11 106) (width 0.25) (layer "F.Cu") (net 5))
 (segment (start 225.301 90.601) (end 224.7 90) (width 0.6) (layer "F.Cu") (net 5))
 (segment (start 203.65 85.35) (end 208 85.35) (width 0.6) (layer "F.Cu") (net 5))
 (segment (start 225.101 88.899) (end 224 90) (width 0.6) (layer "F.Cu") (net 5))
 (segment (start 203.35 104.54) (end 203.753 104.54) (width 0.6) (layer "F.Cu") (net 5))
 (segment (start 203.753 104.54) (end 204.8 104.54) (width 0.6) (layer "F.Cu") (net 5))
 (segment (start 224.2 82.998) (end 225.101 83.899) (width 0.6) (layer "F.Cu") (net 5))
 (segment (start 217.201 93.201) (end 224.809424 93.201) (width 0.6) (layer "F.Cu") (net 5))
 (segment (start 208 85.35) (end 208 83.3) (width 0.6) (layer "F.Cu") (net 5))
 (segment (start 204.8 104.54) (end 209.301 100.039) (width 0.6) (layer "F.Cu") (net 5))
 (segment (start 209.301 100.039) (end 209.301 88.1766) (width 0.6) (layer "F.Cu") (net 5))
 (segment (start 216.54 111.46) (end 216.54 111.638) (width 0.6) (layer "F.Cu") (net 5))
 (segment (start 216.54 112) (end 222.54 106) (width 0.6) (layer "F.Cu") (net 5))
 (segment (start 216.54 112) (end 215.264 113.276) (width 0.6) (layer "F.Cu") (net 5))
 (segment (start 208 83.3) (end 208.302 82.998) (width 0.6) (layer "F.Cu") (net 5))
 (segment (start 205.1065 105.8935) (end 205.1065 105.9965) (width 0.25) (layer "F.Cu") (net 5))
 (segment (start 199.65 88.35) (end 200.65 88.35) (width 0.6) (layer "F.Cu") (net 5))
 (segment (start 225.101 83.899) (end 225.101 86.101) (width 0.6) (layer "F.Cu") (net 5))
 (segment (start 194.7 83.4) (end 199.65 88.35) (width 0.6) (layer "F.Cu") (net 5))
 (segment (start 200.65 88.35) (end 203.249 88.35) (width 0.6) (layer "F.Cu") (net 5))
 (segment (start 222.54 106) (end 223 106) (width 0.25) (layer "F.Cu") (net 5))
 (segment (start 216.54 112) (end 215.804537 112) (width 0.25) (layer "F.Cu") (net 5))
 (segment (start 208.302 82.998) (end 224.2 82.998) (width 0.6) (layer "F.Cu") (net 5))
 (segment (start 194.7 76) (end 194.7 83.4) (width 0.6) (layer "F.Cu") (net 5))
 (segment (start 216 92) (end 217.201 93.201) (width 0.6) (layer "F.Cu") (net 5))
 (segment (start 208.723 87.599) (end 204 87.599) (width 0.6) (layer "F.Cu") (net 5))
 (segment (start 224.7 90) (end 224 90) (width 0.6) (layer "F.Cu") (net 5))
 (segment (start 200.65 88.35) (end 203.65 85.35) (width 0.6) (layer "F.Cu") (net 5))
 (segment (start 225.301 92.709424) (end 225.301 90.601) (width 0.6) (layer "F.Cu") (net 5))
 (segment (start 209.301 88.1766) (end 208.723 87.599) (width 0.6) (layer "F.Cu") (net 5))
 (segment (start 203.249 88.35) (end 204 87.599) (width 0.6) (layer "F.Cu") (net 5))
 (segment (start 204 87.599) (end 203.701 87.599) (width 0.6) (layer "F.Cu") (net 5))
 (segment (start 203.753 104.54) (end 205.1065 105.8935) (width 0.6) (layer "F.Cu") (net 5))
 (segment (start 216.54 112) (end 216.54 111.638) (width 0.25) (layer "F.Cu") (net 5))
 (segment (start 224.809424 93.201) (end 225.301 92.709424) (width 0.6) (layer "F.Cu") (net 5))
 (segment (start 187.7 86.9) (end 188 87.2) (width 0.6) (layer "F.Cu") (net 11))
 (segment (start 187.7 76) (end 187.7 86.9) (width 0.6) (layer "F.Cu") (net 11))
 (segment (start 217.989576 96) (end 214 92.010424) (width 0.6) (layer "F.Cu") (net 9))
 (segment (start 189 98) (end 188.3 98) (width 0.6) (layer "F.Cu") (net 9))
 (segment (start 219.08 111.92) (end 219.08 112) (width 0.6) (layer "F.Cu") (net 9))
 (segment (start 217.101 83.899) (end 213 83.899) (width 0.6) (layer "F.Cu") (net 9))
 (segment (start 188.3 98) (end 187.699 98.601) (width 0.6) (layer "F.Cu") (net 9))
 (segment (start 224.326 105.251) (end 223 103.925) (width 0.6) (layer "F.Cu") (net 9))
 (segment (start 188 97) (end 189 98) (width 0.6) (layer "F.Cu") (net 9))
 (segment (start 224 85) (end 218.202 85) (width 0.6) (layer "F.Cu") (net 9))
 (segment (start 214 87.598) (end 215.497 86.101) (width 0.6) (layer "F.Cu") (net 9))
 (segment (start 210.65 86.249) (end 210.65 100.73) (width 0.6) (layer "F.Cu") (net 9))
 (segment (start 219.08 112) (end 224.326 106.754) (width 0.6) (layer "F.Cu") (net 9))
 (segment (start 188 94) (end 188 97) (width 0.6) (layer "F.Cu") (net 9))
 (segment (start 214 92.010424) (end 214 87.598) (width 0.6) (layer "F.Cu") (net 9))
 (segment (start 187.699 113.699) (end 188.352 114.352) (width 0.6) (layer "F.Cu") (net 9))
 (segment (start 224.326 106.754) (end 224.326 105.251) (width 0.6) (layer "F.Cu") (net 9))
 (segment (start 223 96) (end 217.989576 96) (width 0.6) (layer "F.Cu") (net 9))
 (segment (start 223 103.925) (end 223 96) (width 0.6) (layer "F.Cu") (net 9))
 (segment (start 218.202 85) (end 217.101 83.899) (width 0.6) (layer "F.Cu") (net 9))
 (segment (start 188.352 114.352) (end 216.728 114.352) (width 0.6) (layer "F.Cu") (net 9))
 (segment (start 215.497 86.101) (end 222.899 86.101) (width 0.6) (layer "F.Cu") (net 9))
 (segment (start 222.899 86.101) (end 224 85) (width 0.6) (layer "F.Cu") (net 9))
 (segment (start 216.728 114.352) (end 219.08 112) (width 0.6) (layer "F.Cu") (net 9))
 (segment (start 213 83.899) (end 210.65 86.249) (width 0.6) (layer "F.Cu") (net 9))
 (segment (start 187.699 98.601) (end 187.699 113.699) (width 0.6) (layer "F.Cu") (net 9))
 (segment (start 196 90) (end 196 89.9896) (width 0.6) (layer "F.Cu") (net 12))
 (segment (start 193.291 88.699) (end 190.301 91.6886) (width 0.6) (layer "F.Cu") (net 12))
 (segment (start 190.301 99.399) (end 189.7 100) (width 0.6) (layer "F.Cu") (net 12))
 (segment (start 198 90) (end 199.65 91.65) (width 0.6) (layer "F.Cu") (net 12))
 (segment (start 196 90) (end 198 90) (width 0.6) (layer "F.Cu") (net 12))
 (segment (start 190.301 98.7094) (end 190.301 76.601) (width 0.6) (layer "F.Cu") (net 12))
 (segment (start 196 89.9896) (end 194.709 88.699) (width 0.6) (layer "F.Cu") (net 12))
 (segment (start 194.709 88.699) (end 193.291 88.699) (width 0.6) (layer "F.Cu") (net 12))
 (segment (start 190.301 76.601) (end 190.2 76.5) (width 0.6) (layer "F.Cu") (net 12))
 (segment (start 189.7 100) (end 189 100) (width 0.6) (layer "F.Cu") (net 12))
 (segment (start 190.301 91.6886) (end 190.301 99.399) (width 0.6) (layer "F.Cu") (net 12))
 (segment (start 198.927 89.401) (end 192.2 82.6744) (width 0.6) (layer "F.Cu") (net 2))
 (segment (start 208 91) (end 208 88.65) (width 0.6) (layer "F.Cu") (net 2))
 (segment (start 192.2 82.6744) (end 192.2 76.5) (width 0.6) (layer "F.Cu") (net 2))
 (segment (start 207.249 89.401) (end 198.927 89.401) (width 0.6) (layer "F.Cu") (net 2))
 (segment (start 208 88.65) (end 207.249 89.401) (width 0.6) (layer "F.Cu") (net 2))
 (segment (start 224 92) (end 223.3 92) (width 0.6) (layer "F.Cu") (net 10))
 (segment (start 223.3 92) (end 222.699 91.399) (width 0.6) (layer "F.Cu") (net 10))
 (segment (start 222.699 89.101) (end 224 87.8) (width 0.6) (layer "F.Cu") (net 10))
 (segment (start 222.699 91.399) (end 222.699 89.101) (width 0.6) (layer "F.Cu") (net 10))
 (segment (start 210.65 104.54) (end 210.65 111.19) (width 0.6) (layer "F.Cu") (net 6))
 (segment (start 210.65 111.19) (end 211.46 112) (width 0.6) (layer "F.Cu") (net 6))
 (segment (start 194 90) (end 194 94.1) (width 0.6) (layer "F.Cu") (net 4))
 (segment (start 194 94.1) (end 194 107.462) (width 0.6) (layer "F.Cu") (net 4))
 (segment (start 203.35 102) (end 204.453 102) (width 0.6) (layer "F.Cu") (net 4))
 (segment (start 205 98) (end 197.9 98) (width 0.6) (layer "F.Cu") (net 4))
 (segment (start 206.726 99.7264) (end 205 98) (width 0.6) (layer "F.Cu") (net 4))
 (segment (start 194.769 108.231) (end 194.769 112.601) (width 0.6) (layer "F.Cu") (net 4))
 (segment (start 194 90) (end 193.899 89.899) (width 0.6) (layer "F.Cu") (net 4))
 (segment (start 194.769 112.601) (end 195.619 113.451) (width 0.6) (layer "F.Cu") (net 4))
 (segment (start 204.453 102) (end 206.726 99.7264) (width 0.6) (layer "F.Cu") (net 4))
 (segment (start 195.619 113.451) (end 202.389 113.451) (width 0.6) (layer "F.Cu") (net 4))
 (segment (start 202.389 113.451) (end 203.84 112) (width 0.6) (layer "F.Cu") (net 4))
 (segment (start 197.9 98) (end 194 94.1) (width 0.6) (layer "F.Cu") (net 4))
 (segment (start 194 107.462) (end 194.769 108.231) (width 0.6) (layer "F.Cu") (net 4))
 (segment (start 210.65 102) (end 209 102) (width 0.6) (layer "F.Cu") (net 8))
 (segment (start 206.38 104.62) (end 206.38 112) (width 0.6) (layer "F.Cu") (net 8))
 (segment (start 209 102) (end 206.38 104.62) (width 0.6) (layer "F.Cu") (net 8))
 (segment (start 198.76 103.87) (end 201.9 100.73) (width 0.6) (layer "F.Cu") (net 3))
 (segment (start 201.9 100.73) (end 203.35 100.73) (width 0.6) (layer "F.Cu") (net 3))
 (segment (start 198.76 112) (end 198.76 103.87) (width 0.6) (layer "F.Cu") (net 3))
 (segment (start 208 99.727) (end 204.457 103.27) (width 0.6) (layer "F.Cu") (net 1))
 (segment (start 201.3 103.87) (end 201.3 112) (width 0.6) (layer "F.Cu") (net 1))
 (segment (start 208 93) (end 208 99.727) (width 0.6) (layer "F.Cu") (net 1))
 (segment (start 204.457 103.27) (end 203.35 103.27) (width 0.6) (layer "F.Cu") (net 1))
 (segment (start 201.9 103.27) (end 201.3 103.87) (width 0.6) (layer "F.Cu") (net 1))
 (segment (start 203.35 103.27) (end 201.9 103.27) (width 0.6) (layer "F.Cu") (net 1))
 (segment (start 209.543 103.27) (end 208.92 103.893) (width 0.6) (layer "F.Cu") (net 7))
 (segment (start 211.757 103.27) (end 210.65 103.27) (width 0.6) (layer "F.Cu") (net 7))
 (segment (start 208.92 103.893) (end 208.92 112) (width 0.6) (layer "F.Cu") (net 7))
 (segment (start 212.101 102.926) (end 211.757 103.27) (width 0.6) (layer "F.Cu") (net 7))
 (segment (start 212.101 86.899) (end 212.101 102.926) (width 0.6) (layer "F.Cu") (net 7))
 (segment (start 210.65 103.27) (end 209.543 103.27) (width 0.6) (layer "F.Cu") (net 7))
 (segment (start 216 85) (end 214 85) (width 0.6) (layer "F.Cu") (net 7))
 (segment (start 214 85) (end 212.101 86.899) (width 0.6) (layer "F.Cu") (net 7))
 (segment (start 216 90) (end 216 87.8) (width 0.6) (layer "F.Cu") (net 13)))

